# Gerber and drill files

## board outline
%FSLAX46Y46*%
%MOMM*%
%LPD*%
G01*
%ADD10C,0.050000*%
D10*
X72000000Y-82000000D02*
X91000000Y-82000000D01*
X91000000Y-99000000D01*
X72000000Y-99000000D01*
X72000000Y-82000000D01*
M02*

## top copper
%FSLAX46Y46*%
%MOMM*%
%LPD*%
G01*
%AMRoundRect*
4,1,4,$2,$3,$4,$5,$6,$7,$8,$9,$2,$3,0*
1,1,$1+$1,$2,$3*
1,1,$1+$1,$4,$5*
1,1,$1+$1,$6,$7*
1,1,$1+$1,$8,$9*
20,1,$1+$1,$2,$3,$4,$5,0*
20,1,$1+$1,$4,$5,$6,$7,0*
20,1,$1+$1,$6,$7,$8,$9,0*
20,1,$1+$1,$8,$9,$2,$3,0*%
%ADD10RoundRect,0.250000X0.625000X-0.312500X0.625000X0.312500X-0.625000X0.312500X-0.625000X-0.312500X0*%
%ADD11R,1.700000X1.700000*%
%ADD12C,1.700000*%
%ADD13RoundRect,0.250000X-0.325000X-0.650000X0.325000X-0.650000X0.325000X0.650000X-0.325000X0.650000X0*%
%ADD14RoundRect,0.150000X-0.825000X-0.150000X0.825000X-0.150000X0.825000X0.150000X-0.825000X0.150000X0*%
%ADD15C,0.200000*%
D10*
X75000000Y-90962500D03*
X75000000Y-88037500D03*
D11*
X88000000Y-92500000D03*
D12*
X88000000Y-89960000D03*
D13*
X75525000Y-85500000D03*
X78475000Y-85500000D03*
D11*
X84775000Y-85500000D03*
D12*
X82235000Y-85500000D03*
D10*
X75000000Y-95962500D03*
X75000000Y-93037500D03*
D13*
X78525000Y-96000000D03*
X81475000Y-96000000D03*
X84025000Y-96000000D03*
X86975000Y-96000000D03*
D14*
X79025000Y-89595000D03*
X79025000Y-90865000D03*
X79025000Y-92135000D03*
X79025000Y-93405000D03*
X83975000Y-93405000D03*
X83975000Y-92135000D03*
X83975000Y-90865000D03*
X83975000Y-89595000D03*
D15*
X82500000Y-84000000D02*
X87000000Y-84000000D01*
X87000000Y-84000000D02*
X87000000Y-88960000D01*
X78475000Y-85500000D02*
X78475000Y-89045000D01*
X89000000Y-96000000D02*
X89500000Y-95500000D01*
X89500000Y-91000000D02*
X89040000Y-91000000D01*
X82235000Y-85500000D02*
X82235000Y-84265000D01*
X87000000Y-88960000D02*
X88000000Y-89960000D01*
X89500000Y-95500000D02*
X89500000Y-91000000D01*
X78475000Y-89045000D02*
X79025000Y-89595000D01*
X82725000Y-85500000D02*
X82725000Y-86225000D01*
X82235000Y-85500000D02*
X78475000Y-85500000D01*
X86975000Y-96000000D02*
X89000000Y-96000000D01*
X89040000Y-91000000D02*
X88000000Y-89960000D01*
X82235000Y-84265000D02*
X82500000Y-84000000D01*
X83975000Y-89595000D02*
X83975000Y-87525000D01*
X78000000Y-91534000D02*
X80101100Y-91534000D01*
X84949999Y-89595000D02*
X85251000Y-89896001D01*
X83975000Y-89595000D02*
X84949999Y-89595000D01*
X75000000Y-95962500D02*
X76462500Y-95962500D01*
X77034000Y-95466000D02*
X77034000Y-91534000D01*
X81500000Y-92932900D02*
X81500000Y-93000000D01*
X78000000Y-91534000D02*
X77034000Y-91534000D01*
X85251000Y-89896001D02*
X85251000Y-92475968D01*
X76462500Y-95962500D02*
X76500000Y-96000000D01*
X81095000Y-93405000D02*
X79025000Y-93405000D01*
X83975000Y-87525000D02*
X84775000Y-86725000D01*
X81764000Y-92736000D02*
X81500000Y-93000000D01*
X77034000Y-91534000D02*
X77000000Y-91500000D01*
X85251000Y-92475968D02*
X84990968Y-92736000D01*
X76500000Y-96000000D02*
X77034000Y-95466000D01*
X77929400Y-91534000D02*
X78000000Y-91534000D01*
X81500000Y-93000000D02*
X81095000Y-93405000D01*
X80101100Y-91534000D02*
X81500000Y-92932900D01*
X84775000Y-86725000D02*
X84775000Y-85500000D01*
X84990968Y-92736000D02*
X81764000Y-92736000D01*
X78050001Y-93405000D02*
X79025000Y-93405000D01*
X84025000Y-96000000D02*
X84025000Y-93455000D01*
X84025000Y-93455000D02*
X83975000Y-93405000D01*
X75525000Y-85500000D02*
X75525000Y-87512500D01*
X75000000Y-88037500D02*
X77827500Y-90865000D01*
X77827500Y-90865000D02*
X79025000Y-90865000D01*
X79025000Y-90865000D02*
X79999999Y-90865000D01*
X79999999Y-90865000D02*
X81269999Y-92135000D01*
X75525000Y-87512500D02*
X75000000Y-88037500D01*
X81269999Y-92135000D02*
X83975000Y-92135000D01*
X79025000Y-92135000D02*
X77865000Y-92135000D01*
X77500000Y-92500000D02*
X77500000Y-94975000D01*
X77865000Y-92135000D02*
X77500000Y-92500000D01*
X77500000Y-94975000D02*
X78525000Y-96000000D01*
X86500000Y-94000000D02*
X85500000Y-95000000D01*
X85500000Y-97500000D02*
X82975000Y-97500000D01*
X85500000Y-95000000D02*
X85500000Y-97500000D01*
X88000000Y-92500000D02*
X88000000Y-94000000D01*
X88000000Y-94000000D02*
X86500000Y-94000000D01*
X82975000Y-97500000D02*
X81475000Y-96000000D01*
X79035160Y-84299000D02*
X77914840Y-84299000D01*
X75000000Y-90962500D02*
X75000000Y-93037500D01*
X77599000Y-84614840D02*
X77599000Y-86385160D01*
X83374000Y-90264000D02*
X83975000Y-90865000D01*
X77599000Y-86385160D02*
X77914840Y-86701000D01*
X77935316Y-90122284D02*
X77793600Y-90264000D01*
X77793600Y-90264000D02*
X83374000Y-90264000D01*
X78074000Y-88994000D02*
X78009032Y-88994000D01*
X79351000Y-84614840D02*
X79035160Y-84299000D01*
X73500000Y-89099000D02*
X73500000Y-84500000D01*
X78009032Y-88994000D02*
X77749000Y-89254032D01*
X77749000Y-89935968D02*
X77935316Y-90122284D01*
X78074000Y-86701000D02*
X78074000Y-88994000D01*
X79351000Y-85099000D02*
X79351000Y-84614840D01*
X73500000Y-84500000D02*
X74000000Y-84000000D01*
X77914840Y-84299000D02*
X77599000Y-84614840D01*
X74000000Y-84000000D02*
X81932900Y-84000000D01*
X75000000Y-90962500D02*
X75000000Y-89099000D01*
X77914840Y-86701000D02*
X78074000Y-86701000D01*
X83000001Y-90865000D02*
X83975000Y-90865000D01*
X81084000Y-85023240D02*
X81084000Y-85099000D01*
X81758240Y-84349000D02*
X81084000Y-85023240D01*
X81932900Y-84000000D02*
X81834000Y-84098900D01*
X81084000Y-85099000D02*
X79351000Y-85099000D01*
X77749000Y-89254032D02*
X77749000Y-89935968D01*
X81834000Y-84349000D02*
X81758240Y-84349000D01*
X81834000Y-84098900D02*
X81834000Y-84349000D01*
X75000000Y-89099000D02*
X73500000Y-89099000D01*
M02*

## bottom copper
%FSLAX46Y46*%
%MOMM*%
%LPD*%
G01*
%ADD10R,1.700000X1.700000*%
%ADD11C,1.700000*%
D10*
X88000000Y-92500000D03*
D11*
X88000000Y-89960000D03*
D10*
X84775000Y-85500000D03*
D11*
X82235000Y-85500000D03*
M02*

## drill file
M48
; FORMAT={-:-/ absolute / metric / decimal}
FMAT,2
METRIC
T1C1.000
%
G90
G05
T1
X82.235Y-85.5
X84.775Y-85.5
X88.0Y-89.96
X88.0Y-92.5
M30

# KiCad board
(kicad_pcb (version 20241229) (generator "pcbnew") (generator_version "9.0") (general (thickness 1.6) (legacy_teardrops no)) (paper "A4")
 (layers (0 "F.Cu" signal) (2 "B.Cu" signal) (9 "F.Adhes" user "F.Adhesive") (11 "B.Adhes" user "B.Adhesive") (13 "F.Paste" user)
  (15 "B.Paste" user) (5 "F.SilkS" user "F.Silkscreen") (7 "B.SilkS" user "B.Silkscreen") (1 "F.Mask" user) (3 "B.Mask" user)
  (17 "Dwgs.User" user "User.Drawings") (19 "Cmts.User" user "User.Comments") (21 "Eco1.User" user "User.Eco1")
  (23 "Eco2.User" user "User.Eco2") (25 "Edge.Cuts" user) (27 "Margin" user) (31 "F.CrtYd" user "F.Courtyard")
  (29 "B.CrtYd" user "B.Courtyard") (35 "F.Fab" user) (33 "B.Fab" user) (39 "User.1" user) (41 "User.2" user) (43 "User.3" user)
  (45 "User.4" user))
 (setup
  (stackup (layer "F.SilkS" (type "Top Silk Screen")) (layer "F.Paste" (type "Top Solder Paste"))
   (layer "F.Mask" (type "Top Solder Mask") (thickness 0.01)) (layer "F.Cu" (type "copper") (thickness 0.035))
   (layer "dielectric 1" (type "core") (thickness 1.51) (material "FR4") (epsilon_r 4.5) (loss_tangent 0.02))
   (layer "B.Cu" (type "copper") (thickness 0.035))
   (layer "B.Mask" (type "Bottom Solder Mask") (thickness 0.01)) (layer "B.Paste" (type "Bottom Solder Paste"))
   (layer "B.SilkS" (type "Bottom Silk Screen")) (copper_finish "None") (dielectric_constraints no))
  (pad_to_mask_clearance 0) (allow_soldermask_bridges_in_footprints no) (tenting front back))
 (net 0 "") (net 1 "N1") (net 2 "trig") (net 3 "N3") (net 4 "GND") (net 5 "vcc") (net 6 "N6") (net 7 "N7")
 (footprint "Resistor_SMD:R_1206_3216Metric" (layer "F.Cu") (at 75 89.5 90)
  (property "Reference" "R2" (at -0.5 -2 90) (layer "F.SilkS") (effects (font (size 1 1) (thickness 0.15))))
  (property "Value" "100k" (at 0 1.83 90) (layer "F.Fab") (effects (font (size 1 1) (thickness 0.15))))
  (pad "1" smd roundrect (at -1.4625 0 90) (size 1.125 1.75) (layers "F.Cu" "F.Mask" "F.Paste") (roundrect_rratio 0.222222) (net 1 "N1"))
  (pad "2" smd roundrect (at 1.4625 0 90) (size 1.125 1.75) (layers "F.Cu" "F.Mask" "F.Paste") (roundrect_rratio 0.222222) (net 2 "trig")))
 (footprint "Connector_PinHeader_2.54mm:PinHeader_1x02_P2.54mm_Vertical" (layer "F.Cu") (at 88 92.5 180)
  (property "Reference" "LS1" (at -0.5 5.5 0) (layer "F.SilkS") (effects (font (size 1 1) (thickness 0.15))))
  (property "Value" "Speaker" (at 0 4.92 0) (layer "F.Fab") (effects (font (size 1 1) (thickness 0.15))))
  (pad "1" thru_hole rect (at 0 0 180) (size 1.7 1.7) (drill 1) (layers "*.Cu" "*.Mask") (remove_unused_layers no) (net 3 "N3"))
  (pad "2" thru_hole circle (at 0 2.54 180) (size 1.7 1.7) (drill 1) (layers "*.Cu" "*.Mask") (remove_unused_layers no) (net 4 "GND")))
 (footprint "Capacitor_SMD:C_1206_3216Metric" (layer "F.Cu") (at 77 85.5)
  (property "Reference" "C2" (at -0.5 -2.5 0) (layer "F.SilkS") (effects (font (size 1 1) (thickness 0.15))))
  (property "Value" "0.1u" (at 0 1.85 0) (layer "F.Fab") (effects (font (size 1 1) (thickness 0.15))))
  (pad "1" smd roundrect (at -1.475 0) (size 1.15 1.8) (layers "F.Cu" "F.Mask" "F.Paste") (roundrect_rratio 0.217391) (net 2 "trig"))
  (pad "2" smd roundrect (at 1.475 0) (size 1.15 1.8) (layers "F.Cu" "F.Mask" "F.Paste") (roundrect_rratio 0.217391) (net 4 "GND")))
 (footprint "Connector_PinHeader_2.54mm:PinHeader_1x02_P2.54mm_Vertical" (layer "F.Cu") (at 84.775 85.5 -90)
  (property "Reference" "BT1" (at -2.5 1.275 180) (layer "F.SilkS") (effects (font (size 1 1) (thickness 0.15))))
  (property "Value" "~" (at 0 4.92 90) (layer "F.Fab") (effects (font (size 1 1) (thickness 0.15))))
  (pad "1" thru_hole rect (at 0 0 270) (size 1.7 1.7) (drill 1) (layers "*.Cu" "*.Mask") (remove_unused_layers no) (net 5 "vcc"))
  (pad "2" thru_hole circle (at 0 2.54 270) (size 1.7 1.7) (drill 1) (layers "*.Cu" "*.Mask") (remove_unused_layers no) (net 4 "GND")))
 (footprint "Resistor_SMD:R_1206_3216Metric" (layer "F.Cu") (at 75 94.5 90)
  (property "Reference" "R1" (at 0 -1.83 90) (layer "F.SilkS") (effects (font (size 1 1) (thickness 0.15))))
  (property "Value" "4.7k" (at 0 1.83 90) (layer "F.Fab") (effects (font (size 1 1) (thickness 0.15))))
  (pad "1" smd roundrect (at -1.4625 0 90) (size 1.125 1.75) (layers "F.Cu" "F.Mask" "F.Paste") (roundrect_rratio 0.222222) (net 5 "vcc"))
  (pad "2" smd roundrect (at 1.4625 0 90) (size 1.125 1.75) (layers "F.Cu" "F.Mask" "F.Paste") (roundrect_rratio 0.222222) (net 1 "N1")))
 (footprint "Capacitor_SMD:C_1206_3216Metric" (layer "F.Cu") (at 80 96)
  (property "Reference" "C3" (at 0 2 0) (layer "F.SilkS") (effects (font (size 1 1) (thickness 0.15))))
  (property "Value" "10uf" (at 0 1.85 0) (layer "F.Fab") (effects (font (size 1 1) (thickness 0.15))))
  (pad "1" smd roundrect (at -1.475 0) (size 1.15 1.8) (layers "F.Cu" "F.Mask" "F.Paste") (roundrect_rratio 0.217391) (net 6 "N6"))
  (pad "2" smd roundrect (at 1.475 0) (size 1.15 1.8) (layers "F.Cu" "F.Mask" "F.Paste") (roundrect_rratio 0.217391) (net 3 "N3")))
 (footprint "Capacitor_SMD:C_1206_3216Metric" (layer "F.Cu") (at 85.5 96)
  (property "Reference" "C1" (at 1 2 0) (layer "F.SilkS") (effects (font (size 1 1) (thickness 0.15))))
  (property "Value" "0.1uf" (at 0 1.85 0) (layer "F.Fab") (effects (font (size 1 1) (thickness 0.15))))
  (pad "1" smd roundrect (at -1.475 0) (size 1.15 1.8) (layers "F.Cu" "F.Mask" "F.Paste") (roundrect_rratio 0.217391) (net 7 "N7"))
  (pad "2" smd roundrect (at 1.475 0) (size 1.15 1.8) (layers "F.Cu" "F.Mask" "F.Paste") (roundrect_rratio 0.217391) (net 4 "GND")))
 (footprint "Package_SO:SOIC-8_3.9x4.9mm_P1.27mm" (layer "F.Cu") (at 81.5 91.5)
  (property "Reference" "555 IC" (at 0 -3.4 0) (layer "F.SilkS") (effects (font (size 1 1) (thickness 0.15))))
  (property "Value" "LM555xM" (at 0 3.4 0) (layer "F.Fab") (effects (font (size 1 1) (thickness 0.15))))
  (pad "1" smd roundrect (at -2.475 -1.905) (size 1.95 0.6) (layers "F.Cu" "F.Mask" "F.Paste") (roundrect_rratio 0.25) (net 4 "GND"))
  (pad "2" smd roundrect (at -2.475 -0.635) (size 1.95 0.6) (layers "F.Cu" "F.Mask" "F.Paste") (roundrect_rratio 0.25) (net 2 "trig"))
  (pad "3" smd roundrect (at -2.475 0.635) (size 1.95 0.6) (layers "F.Cu" "F.Mask" "F.Paste") (roundrect_rratio 0.25) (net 6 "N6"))
  (pad "4" smd roundrect (at -2.475 1.905) (size 1.95 0.6) (layers "F.Cu" "F.Mask" "F.Paste") (roundrect_rratio 0.25) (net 5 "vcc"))
  (pad "5" smd roundrect (at 2.475 1.905) (size 1.95 0.6) (layers "F.Cu" "F.Mask" "F.Paste") (roundrect_rratio 0.25) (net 7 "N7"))
  (pad "6" smd roundrect (at 2.475 0.635) (size 1.95 0.6) (layers "F.Cu" "F.Mask" "F.Paste") (roundrect_rratio 0.25) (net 2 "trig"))
  (pad "7" smd roundrect (at 2.475 -0.635) (size 1.95 0.6) (layers "F.Cu" "F.Mask" "F.Paste") (roundrect_rratio 0.25) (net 1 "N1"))
  (pad "8" smd roundrect (at 2.475 -1.905) (size 1.95 0.6) (layers "F.Cu" "F.Mask" "F.Paste") (roundrect_rratio 0.25) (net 5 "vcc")))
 (gr_rect (start 72 82) (end 91 99) (stroke (width 0.05) (type default)) (fill no) (layer "Edge.Cuts"))
 (segment (start 82.5 84) (end 87 84) (width 0.2) (layer "F.Cu") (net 4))
 (segment (start 87 84) (end 87 88.96) (width 0.2) (layer "F.Cu") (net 4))
 (segment (start 78.475 85.5) (end 78.475 89.045) (width 0.2) (layer "F.Cu") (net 4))
 (segment (start 89 96) (end 89.5 95.5) (width 0.2) (layer "F.Cu") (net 4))
 (segment (start 89.5 91) (end 89.04 91) (width 0.2) (layer "F.Cu") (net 4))
 (segment (start 82.235 85.5) (end 82.235 84.265) (width 0.2) (layer "F.Cu") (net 4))
 (segment (start 87 88.96) (end 88 89.96) (width 0.2) (layer "F.Cu") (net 4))
 (segment (start 89.5 95.5) (end 89.5 91) (width 0.2) (layer "F.Cu") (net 4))
 (segment (start 78.475 89.045) (end 79.025 89.595) (width 0.2) (layer "F.Cu") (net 4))
 (segment (start 82.725 85.5) (end 82.725 86.225) (width 0.2) (layer "F.Cu") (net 4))
 (segment (start 82.235 85.5) (end 78.475 85.5) (width 0.2) (layer "F.Cu") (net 4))
 (segment (start 86.975 96) (end 89 96) (width 0.2) (layer "F.Cu") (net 4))
 (segment (start 89.04 91) (end 88 89.96) (width 0.2) (layer "F.Cu") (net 4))
 (segment (start 82.235 84.265) (end 82.5 84) (width 0.2) (layer "F.Cu") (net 4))
 (segment (start 83.975 89.595) (end 83.975 87.525) (width 0.2) (layer "F.Cu") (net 5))
 (segment (start 78 91.534) (end 80.1011 91.534) (width 0.2) (layer "F.Cu") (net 5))
 (segment (start 84.949999 89.595) (end 85.251 89.896001) (width 0.2) (layer "F.Cu") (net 5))
 (segment (start 83.975 89.595) (end 84.949999 89.595) (width 0.2) (layer "F.Cu") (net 5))
 (segment (start 75 95.9625) (end 76.4625 95.9625) (width 0.2) (layer "F.Cu") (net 5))
 (segment (start 77.034 95.466) (end 77.034 91.534) (width 0.2) (layer "F.Cu") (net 5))
 (segment (start 81.5 92.9329) (end 81.5 93) (width 0.2) (layer "F.Cu") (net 5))
 (segment (start 78 91.534) (end 77.034 91.534) (width 0.2) (layer "F.Cu") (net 5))
 (segment (start 85.251 89.896001) (end 85.251 92.475968) (width 0.2) (layer "F.Cu") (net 5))
 (segment (start 76.4625 95.9625) (end 76.5 96) (width 0.2) (layer "F.Cu") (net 5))
 (segment (start 81.095 93.405) (end 79.025 93.405) (width 0.2) (layer "F.Cu") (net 5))
 (segment (start 83.975 87.525) (end 84.775 86.725) (width 0.2) (layer "F.Cu") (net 5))
 (segment (start 81.764 92.736) (end 81.5 93) (width 0.2) (layer "F.Cu") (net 5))
 (segment (start 77.034 91.534) (end 77 91.5) (width 0.2) (layer "F.Cu") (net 5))
 (segment (start 85.251 92.475968) (end 84.990968 92.736) (width 0.2) (layer "F.Cu") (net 5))
 (segment (start 76.5 96) (end 77.034 95.466) (width 0.2) (layer "F.Cu") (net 5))
 (segment (start 77.9294 91.534) (end 78 91.534) (width 0.2) (layer "F.Cu") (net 5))
 (segment (start 81.5 93) (end 81.095 93.405) (width 0.2) (layer "F.Cu") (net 5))
 (segment (start 80.1011 91.534) (end 81.5 92.9329) (width 0.2) (layer "F.Cu") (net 5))
 (segment (start 84.775 86.725) (end 84.775 85.5) (width 0.2) (layer "F.Cu") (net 5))
 (segment (start 84.990968 92.736) (end 81.764 92.736) (width 0.2) (layer "F.Cu") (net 5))
 (segment (start 78.050001 93.405) (end 79.025 93.405) (width 0.2) (layer "F.Cu") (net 5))
 (segment (start 84.025 96) (end 84.025 93.455) (width 0.2) (layer "F.Cu") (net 7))
 (segment (start 84.025 93.455) (end 83.975 93.405) (width 0.2) (layer "F.Cu") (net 7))
 (segment (start 75.525 85.5) (end 75.525 87.5125) (width 0.2) (layer "F.Cu") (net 2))
 (segment (start 75 88.0375) (end 77.8275 90.865) (width 0.2) (layer "F.Cu") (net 2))
 (segment (start 77.8275 90.865) (end 79.025 90.865) (width 0.2) (layer "F.Cu") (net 2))
 (segment (start 79.025 90.865) (end 79.999999 90.865) (width 0.2) (layer "F.Cu") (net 2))
 (segment (start 79.999999 90.865) (end 81.269999 92.135) (width 0.2) (layer "F.Cu") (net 2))
 (segment (start 75.525 87.5125) (end 75 88.0375) (width 0.2) (layer "F.Cu") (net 2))
 (segment (start 81.269999 92.135) (end 83.975 92.135) (width 0.2) (layer "F.Cu") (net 2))
 (segment (start 79.025 92.135) (end 77.865 92.135) (width 0.2) (layer "F.Cu") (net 6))
 (segment (start 77.5 92.5) (end 77.5 94.975) (width 0.2) (layer "F.Cu") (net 6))
 (segment (start 77.865 92.135) (end 77.5 92.5) (width 0.2) (layer "F.Cu") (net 6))
 (segment (start 77.5 94.975) (end 78.525 96) (width 0.2) (layer "F.Cu") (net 6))
 (segment (start 86.5 94) (end 85.5 95) (width 0.2) (layer "F.Cu") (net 3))
 (segment (start 85.5 97.5) (end 82.975 97.5) (width 0.2) (layer "F.Cu") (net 3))
 (segment (start 85.5 95) (end 85.5 97.5) (width 0.2) (layer "F.Cu") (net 3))
 (segment (start 88 92.5) (end 88 94) (width 0.2) (layer "F.Cu") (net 3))
 (segment (start 88 94) (end 86.5 94) (width 0.2) (layer "F.Cu") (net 3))
 (segment (start 82.975 97.5) (end 81.475 96) (width 0.2) (layer "F.Cu") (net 3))
 (segment (start 79.03516 84.299) (end 77.91484 84.299) (width 0.2) (layer "F.Cu") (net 1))
 (segment (start 75 90.9625) (end 75 93.0375) (width 0.2) (layer "F.Cu") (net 1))
 (segment (start 77.599 84.61484) (end 77.599 86.38516) (width 0.2) (layer "F.Cu") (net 1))
 (segment (start 83.374 90.264) (end 83.975 90.865) (width 0.2) (layer "F.Cu") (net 1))
 (segment (start 77.599 86.38516) (end 77.91484 86.701) (width 0.2) (layer "F.Cu") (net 1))
 (segment (start 77.935316 90.122284) (end 77.7936 90.264) (width 0.2) (layer "F.Cu") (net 1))
 (segment (start 77.7936 90.264) (end 83.374 90.264) (width 0.2) (layer "F.Cu") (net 1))
 (segment (start 78.074 88.994) (end 78.009032 88.994) (width 0.2) (layer "F.Cu") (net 1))
 (segment (start 79.351 84.61484) (end 79.03516 84.299) (width 0.2) (layer "F.Cu") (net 1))
 (segment (start 73.5 89.099) (end 73.5 84.5) (width 0.2) (layer "F.Cu") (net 1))
 (segment (start 78.009032 88.994) (end 77.749 89.254032) (width 0.2) (layer "F.Cu") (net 1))
 (segment (start 77.749 89.935968) (end 77.935316 90.122284) (width 0.2) (layer "F.Cu") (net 1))
 (segment (start 78.074 86.701) (end 78.074 88.994) (width 0.2) (layer "F.Cu") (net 1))
 (segment (start 79.351 85.099) (end 79.351 84.61484) (width 0.2) (layer "F.Cu") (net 1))
 (segment (start 73.5 84.5) (end 74 84) (width 0.2) (layer "F.Cu") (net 1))
 (segment (start 77.91484 84.299) (end 77.599 84.61484) (width 0.2) (layer "F.Cu") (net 1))
 (segment (start 74 84) (end 81.9329 84) (width 0.2) (layer "F.Cu") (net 1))
 (segment (start 75 90.9625) (end 75 89.099) (width 0.2) (layer "F.Cu") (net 1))
 (segment (start 77.91484 86.701) (end 78.074 86.701) (width 0.2) (layer "F.Cu") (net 1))
 (segment (start 83.000001 90.865) (end 83.975 90.865) (width 0.2) (layer "F.Cu") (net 1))
 (segment (start 81.084 85.02324) (end 81.084 85.099) (width 0.2) (layer "F.Cu") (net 1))
 (segment (start 81.75824 84.349) (end 81.084 85.02324) (width 0.2) (layer "F.Cu") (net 1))
 (segment (start 81.9329 84) (end 81.834 84.0989) (width 0.2) (layer "F.Cu") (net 1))
 (segment (start 81.084 85.099) (end 79.351 85.099) (width 0.2) (layer "F.Cu") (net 1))
 (segment (start 77.749 89.254032) (end 77.749 89.935968) (width 0.2) (layer "F.Cu") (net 1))
 (segment (start 81.834 84.349) (end 81.75824 84.349) (width 0.2) (layer "F.Cu") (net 1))
 (segment (start 81.834 84.0989) (end 81.834 84.349) (width 0.2) (layer "F.Cu") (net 1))
 (segment (start 75 89.099) (end 73.5 89.099) (width 0.2) (layer "F.Cu") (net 1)))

